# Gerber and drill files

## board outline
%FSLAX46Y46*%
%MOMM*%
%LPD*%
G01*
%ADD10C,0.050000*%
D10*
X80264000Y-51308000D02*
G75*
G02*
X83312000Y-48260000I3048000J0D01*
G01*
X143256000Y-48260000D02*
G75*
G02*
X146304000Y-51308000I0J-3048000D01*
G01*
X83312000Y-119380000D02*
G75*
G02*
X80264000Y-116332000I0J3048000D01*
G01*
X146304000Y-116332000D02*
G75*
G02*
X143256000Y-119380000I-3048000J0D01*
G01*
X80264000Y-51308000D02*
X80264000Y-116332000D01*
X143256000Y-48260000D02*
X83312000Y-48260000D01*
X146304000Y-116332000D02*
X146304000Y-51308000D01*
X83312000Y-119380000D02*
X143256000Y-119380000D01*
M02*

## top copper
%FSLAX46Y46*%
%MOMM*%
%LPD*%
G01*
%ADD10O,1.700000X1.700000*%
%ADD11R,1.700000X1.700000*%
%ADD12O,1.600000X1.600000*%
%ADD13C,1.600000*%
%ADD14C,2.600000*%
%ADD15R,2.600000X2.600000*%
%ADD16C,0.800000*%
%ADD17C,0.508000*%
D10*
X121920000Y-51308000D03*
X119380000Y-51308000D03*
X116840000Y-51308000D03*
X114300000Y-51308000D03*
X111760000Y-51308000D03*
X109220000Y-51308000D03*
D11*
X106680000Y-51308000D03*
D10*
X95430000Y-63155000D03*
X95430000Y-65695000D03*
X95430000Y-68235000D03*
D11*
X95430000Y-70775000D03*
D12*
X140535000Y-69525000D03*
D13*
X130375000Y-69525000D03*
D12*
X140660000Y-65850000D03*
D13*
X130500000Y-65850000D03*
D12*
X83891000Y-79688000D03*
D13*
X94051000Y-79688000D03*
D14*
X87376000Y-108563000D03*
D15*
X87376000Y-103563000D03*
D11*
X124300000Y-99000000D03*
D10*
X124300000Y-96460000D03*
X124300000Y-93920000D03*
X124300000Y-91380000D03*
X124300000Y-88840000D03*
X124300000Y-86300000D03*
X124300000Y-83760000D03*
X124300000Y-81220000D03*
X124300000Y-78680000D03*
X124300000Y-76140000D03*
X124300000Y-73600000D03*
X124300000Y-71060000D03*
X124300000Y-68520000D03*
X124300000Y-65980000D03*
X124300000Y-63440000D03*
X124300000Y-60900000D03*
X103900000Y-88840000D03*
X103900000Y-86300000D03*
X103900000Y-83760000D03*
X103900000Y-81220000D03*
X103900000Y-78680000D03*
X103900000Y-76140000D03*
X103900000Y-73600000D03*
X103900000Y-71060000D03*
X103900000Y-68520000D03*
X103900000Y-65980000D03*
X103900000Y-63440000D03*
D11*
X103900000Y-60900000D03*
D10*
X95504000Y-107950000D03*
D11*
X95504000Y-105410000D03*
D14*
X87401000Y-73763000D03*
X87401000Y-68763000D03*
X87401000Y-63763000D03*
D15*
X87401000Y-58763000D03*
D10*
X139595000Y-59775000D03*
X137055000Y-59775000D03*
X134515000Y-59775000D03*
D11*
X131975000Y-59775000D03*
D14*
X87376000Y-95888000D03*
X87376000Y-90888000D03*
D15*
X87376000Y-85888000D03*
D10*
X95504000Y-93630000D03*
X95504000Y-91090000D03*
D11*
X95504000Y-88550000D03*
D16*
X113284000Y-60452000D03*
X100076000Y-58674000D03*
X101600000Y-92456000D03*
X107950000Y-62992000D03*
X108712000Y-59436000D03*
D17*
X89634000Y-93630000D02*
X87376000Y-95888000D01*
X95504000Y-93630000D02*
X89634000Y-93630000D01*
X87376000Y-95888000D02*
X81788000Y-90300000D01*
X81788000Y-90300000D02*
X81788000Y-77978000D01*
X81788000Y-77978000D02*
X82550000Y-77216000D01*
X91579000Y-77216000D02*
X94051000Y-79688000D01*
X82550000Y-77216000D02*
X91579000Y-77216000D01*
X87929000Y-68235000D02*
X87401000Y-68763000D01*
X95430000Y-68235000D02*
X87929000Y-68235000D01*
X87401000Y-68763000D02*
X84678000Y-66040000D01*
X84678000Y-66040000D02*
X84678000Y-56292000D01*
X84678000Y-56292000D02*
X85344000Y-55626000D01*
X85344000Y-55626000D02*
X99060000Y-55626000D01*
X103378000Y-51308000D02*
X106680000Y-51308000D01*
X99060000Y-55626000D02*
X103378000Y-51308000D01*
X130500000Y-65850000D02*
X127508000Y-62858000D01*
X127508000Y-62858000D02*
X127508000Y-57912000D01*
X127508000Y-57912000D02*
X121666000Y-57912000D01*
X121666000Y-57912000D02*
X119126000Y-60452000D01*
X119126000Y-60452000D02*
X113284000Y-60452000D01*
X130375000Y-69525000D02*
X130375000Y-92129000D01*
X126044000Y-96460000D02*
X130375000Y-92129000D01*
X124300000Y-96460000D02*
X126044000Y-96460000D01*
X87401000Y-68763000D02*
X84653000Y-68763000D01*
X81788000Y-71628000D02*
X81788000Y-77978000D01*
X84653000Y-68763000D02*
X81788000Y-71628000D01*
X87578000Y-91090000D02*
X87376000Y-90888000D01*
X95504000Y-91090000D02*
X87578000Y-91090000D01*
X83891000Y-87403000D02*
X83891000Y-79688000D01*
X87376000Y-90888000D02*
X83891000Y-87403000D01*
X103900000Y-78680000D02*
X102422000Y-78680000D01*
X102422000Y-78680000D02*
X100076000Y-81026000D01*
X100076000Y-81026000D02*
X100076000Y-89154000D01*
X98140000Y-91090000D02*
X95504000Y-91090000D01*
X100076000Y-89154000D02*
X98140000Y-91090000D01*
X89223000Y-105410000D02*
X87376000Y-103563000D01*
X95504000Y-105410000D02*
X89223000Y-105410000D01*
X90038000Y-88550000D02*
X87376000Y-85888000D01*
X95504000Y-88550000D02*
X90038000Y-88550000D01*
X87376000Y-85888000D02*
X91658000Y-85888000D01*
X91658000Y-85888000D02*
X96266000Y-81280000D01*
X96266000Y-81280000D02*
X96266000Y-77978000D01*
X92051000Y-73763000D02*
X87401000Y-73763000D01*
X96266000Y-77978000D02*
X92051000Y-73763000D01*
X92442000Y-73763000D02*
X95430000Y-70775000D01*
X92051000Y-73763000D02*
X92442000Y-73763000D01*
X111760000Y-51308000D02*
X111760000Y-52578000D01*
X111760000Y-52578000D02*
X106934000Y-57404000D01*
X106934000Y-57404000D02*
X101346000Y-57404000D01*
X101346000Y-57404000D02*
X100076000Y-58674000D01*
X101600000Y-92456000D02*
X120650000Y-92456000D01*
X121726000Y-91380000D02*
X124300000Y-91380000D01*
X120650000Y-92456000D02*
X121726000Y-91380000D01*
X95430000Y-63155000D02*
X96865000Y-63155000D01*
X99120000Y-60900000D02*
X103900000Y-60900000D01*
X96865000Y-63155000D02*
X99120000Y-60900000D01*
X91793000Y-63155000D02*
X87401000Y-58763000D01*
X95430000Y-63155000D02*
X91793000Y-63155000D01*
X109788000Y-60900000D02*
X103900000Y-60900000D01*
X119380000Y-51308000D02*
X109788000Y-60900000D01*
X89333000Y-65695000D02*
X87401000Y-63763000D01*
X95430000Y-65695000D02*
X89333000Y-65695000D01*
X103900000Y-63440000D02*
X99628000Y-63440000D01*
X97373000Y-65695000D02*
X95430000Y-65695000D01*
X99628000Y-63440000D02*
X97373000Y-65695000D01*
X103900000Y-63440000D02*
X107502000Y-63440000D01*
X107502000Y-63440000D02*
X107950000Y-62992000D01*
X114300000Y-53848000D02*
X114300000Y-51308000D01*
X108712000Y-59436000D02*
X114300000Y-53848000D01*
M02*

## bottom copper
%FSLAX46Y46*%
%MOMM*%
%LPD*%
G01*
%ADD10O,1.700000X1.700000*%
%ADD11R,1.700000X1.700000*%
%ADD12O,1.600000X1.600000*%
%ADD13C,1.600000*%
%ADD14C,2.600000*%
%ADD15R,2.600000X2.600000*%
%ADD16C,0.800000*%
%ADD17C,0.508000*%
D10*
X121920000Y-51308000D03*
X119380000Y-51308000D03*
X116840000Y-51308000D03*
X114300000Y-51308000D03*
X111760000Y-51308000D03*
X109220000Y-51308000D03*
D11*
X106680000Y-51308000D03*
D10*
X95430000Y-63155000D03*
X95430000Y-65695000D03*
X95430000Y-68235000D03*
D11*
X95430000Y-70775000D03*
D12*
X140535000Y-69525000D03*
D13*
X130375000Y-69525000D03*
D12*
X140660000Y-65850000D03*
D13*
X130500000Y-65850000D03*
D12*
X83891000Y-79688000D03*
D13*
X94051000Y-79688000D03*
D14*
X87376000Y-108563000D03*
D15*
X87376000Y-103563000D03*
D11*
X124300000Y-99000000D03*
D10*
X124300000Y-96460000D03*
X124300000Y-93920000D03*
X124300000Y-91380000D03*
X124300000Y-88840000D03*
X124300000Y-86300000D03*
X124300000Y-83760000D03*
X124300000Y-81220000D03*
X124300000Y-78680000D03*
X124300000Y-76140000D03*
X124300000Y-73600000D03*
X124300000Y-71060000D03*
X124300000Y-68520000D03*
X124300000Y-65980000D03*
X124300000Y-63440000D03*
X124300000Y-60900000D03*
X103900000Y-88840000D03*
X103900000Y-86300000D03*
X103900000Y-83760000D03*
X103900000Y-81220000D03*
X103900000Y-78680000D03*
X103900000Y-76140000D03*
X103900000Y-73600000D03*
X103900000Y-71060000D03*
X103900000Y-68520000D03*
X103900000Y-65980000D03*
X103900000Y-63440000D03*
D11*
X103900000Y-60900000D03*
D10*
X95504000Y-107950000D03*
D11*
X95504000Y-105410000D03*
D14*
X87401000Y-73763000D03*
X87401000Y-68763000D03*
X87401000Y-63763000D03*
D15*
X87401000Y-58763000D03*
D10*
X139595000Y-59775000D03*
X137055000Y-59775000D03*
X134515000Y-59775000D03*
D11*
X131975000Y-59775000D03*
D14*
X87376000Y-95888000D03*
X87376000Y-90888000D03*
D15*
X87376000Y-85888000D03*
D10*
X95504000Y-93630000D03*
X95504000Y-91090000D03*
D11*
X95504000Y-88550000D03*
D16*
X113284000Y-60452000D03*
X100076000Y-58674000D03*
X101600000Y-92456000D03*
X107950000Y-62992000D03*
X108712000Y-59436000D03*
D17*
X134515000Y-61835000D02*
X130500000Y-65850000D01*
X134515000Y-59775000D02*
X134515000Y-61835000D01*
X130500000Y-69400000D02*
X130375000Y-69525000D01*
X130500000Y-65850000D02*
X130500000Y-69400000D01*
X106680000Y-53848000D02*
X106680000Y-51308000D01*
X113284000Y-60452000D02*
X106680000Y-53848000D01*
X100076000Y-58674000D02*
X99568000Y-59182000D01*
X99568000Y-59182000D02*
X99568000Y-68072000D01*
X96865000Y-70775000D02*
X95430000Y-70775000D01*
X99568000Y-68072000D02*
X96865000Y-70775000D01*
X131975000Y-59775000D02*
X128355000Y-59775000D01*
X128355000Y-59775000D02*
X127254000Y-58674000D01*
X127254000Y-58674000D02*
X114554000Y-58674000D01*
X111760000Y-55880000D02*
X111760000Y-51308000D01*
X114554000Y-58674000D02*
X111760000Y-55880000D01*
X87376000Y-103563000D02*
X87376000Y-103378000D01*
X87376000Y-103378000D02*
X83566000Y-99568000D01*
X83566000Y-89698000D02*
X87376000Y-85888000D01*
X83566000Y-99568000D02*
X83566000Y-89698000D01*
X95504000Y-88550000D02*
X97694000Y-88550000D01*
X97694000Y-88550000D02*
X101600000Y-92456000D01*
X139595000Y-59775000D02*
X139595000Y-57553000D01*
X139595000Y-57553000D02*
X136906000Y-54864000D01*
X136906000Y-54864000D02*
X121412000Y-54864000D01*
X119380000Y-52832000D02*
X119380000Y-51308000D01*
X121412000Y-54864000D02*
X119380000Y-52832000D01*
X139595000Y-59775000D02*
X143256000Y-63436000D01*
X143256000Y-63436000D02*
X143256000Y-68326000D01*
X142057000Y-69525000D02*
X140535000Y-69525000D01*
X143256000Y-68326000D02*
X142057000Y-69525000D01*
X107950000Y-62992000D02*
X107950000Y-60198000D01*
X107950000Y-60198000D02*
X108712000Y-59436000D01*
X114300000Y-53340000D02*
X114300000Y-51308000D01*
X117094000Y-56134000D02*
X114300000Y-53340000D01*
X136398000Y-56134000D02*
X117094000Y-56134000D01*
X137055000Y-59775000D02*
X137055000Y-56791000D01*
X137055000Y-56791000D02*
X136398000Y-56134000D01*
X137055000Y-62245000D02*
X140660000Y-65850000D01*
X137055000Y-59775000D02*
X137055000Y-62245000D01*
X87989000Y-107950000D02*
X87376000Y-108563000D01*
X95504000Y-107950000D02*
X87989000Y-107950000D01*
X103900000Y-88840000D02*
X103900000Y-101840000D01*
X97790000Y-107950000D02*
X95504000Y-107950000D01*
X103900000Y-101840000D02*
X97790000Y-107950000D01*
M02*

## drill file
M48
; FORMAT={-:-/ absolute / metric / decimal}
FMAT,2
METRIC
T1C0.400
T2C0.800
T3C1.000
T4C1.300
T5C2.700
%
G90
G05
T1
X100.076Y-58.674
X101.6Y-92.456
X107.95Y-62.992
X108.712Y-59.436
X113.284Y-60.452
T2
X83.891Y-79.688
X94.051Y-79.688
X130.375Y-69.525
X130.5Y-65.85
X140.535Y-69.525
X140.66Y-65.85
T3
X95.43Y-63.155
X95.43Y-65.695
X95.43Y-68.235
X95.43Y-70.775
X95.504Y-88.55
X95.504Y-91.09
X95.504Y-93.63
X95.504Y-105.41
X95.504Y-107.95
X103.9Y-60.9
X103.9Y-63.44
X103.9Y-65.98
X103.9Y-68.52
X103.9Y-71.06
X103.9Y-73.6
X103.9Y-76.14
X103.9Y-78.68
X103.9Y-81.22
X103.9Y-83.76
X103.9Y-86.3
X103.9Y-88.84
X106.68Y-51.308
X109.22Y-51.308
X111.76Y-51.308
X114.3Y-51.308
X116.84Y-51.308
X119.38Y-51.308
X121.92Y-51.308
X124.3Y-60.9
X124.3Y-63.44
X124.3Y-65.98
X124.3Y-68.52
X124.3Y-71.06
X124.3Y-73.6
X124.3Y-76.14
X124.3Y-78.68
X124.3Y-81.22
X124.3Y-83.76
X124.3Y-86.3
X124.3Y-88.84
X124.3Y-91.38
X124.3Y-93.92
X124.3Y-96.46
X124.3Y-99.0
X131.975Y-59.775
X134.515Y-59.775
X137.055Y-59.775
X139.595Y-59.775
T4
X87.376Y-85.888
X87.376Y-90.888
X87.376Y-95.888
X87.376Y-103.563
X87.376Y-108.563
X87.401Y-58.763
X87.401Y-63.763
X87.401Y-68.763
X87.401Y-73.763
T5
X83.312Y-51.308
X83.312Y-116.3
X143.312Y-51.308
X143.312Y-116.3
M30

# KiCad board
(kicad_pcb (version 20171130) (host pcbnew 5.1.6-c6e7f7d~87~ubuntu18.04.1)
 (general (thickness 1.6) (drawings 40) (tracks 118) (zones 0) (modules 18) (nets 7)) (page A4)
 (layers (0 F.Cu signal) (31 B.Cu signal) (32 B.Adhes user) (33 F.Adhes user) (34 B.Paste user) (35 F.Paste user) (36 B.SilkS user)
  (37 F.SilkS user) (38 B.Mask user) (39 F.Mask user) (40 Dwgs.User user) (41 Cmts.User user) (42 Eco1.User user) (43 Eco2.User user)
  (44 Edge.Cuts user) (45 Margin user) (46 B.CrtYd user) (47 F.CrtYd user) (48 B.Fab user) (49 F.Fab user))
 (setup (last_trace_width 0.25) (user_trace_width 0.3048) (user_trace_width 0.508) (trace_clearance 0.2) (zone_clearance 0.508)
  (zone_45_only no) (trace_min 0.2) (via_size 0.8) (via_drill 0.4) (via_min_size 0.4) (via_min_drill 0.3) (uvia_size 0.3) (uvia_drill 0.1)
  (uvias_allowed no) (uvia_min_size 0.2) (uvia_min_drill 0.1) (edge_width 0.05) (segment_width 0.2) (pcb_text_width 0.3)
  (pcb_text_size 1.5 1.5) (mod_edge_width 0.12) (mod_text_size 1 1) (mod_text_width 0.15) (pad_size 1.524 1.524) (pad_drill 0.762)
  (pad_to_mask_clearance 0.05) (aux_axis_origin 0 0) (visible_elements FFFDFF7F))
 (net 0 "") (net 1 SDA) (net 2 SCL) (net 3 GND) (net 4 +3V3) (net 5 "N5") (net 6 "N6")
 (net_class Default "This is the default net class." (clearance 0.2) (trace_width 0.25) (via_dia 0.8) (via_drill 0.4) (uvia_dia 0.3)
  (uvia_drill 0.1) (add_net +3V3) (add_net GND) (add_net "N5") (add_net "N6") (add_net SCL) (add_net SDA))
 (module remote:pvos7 (layer F.Cu) (at 135.89 91.948 90)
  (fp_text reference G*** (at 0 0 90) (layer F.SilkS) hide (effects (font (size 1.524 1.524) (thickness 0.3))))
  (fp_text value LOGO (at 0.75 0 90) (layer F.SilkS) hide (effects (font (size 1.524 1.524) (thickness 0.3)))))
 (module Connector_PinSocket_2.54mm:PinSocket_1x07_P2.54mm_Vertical (layer F.Cu) (at 106.68 51.308 90)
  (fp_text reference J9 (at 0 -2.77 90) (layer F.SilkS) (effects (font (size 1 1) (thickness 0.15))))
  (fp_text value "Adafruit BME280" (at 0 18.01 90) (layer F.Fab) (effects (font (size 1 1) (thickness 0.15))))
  (pad 7 thru_hole oval (at 0 15.24 90) (size 1.7 1.7) (drill 1) (layers *.Cu *.Mask))
  (pad 6 thru_hole oval (at 0 12.7 90) (size 1.7 1.7) (drill 1) (layers *.Cu *.Mask) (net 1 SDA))
  (pad 5 thru_hole oval (at 0 10.16 90) (size 1.7 1.7) (drill 1) (layers *.Cu *.Mask))
  (pad 4 thru_hole oval (at 0 7.62 90) (size 1.7 1.7) (drill 1) (layers *.Cu *.Mask) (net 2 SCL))
  (pad 3 thru_hole oval (at 0 5.08 90) (size 1.7 1.7) (drill 1) (layers *.Cu *.Mask) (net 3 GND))
  (pad 2 thru_hole oval (at 0 2.54 90) (size 1.7 1.7) (drill 1) (layers *.Cu *.Mask))
  (pad 1 thru_hole rect (at 0 0 90) (size 1.7 1.7) (drill 1) (layers *.Cu *.Mask) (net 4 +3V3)))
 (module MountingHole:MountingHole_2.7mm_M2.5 (layer F.Cu) (at 143.312 116.3)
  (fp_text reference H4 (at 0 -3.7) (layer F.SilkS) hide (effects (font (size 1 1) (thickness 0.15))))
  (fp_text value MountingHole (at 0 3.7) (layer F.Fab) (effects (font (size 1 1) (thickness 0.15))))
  (pad 1 np_thru_hole circle (at 0 0) (size 2.7 2.7) (drill 2.7) (layers *.Cu *.Mask)))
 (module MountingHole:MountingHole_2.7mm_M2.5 (layer F.Cu) (at 83.312 116.3)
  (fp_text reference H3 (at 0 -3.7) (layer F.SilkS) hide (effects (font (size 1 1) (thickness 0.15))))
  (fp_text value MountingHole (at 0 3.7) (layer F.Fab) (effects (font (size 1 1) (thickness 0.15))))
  (pad 1 np_thru_hole circle (at 0 0) (size 2.7 2.7) (drill 2.7) (layers *.Cu *.Mask)))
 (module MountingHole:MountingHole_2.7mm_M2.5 (layer F.Cu) (at 143.312 51.308)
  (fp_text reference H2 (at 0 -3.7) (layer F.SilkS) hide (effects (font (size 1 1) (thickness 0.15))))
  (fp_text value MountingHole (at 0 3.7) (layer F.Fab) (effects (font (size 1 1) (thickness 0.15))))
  (pad 1 np_thru_hole circle (at 0 0) (size 2.7 2.7) (drill 2.7) (layers *.Cu *.Mask)))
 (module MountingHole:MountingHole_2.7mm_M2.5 (layer F.Cu) (at 83.312 51.308)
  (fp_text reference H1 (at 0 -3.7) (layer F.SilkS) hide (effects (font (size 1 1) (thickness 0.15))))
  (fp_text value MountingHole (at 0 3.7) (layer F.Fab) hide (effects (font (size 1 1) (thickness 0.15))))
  (pad 1 np_thru_hole circle (at 0 0) (size 2.7 2.7) (drill 2.7) (layers *.Cu *.Mask)))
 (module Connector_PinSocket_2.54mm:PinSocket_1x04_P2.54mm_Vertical (layer F.Cu) (at 95.43 70.775 180)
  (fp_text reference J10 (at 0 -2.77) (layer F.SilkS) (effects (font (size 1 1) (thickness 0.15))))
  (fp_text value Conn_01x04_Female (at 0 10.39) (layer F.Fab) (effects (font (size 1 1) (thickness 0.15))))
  (pad 4 thru_hole oval (at 0 7.62 180) (size 1.7 1.7) (drill 1) (layers *.Cu *.Mask) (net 1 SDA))
  (pad 3 thru_hole oval (at 0 5.08 180) (size 1.7 1.7) (drill 1) (layers *.Cu *.Mask) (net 2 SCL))
  (pad 2 thru_hole oval (at 0 2.54 180) (size 1.7 1.7) (drill 1) (layers *.Cu *.Mask) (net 4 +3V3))
  (pad 1 thru_hole rect (at 0 0 180) (size 1.7 1.7) (drill 1) (layers *.Cu *.Mask) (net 3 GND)))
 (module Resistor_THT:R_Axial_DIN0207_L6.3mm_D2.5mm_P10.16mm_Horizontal (layer F.Cu) (at 130.375 69.525)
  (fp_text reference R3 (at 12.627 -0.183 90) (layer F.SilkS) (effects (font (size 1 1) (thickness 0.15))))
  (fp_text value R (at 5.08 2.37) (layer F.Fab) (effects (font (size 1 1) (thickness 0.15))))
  (pad 2 thru_hole oval (at 10.16 0) (size 1.6 1.6) (drill 0.8) (layers *.Cu *.Mask) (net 1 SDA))
  (pad 1 thru_hole circle (at 0 0) (size 1.6 1.6) (drill 0.8) (layers *.Cu *.Mask) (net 4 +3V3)))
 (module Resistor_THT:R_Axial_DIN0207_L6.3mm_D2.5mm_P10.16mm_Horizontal (layer F.Cu) (at 130.5 65.85)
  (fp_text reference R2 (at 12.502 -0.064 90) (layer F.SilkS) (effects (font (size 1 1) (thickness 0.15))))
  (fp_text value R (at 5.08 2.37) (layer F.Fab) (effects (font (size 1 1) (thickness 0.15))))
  (pad 2 thru_hole oval (at 10.16 0) (size 1.6 1.6) (drill 0.8) (layers *.Cu *.Mask) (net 2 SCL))
  (pad 1 thru_hole circle (at 0 0) (size 1.6 1.6) (drill 0.8) (layers *.Cu *.Mask) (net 4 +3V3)))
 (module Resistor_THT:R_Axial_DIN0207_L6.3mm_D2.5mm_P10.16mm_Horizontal (layer F.Cu) (at 94.051 79.688 180)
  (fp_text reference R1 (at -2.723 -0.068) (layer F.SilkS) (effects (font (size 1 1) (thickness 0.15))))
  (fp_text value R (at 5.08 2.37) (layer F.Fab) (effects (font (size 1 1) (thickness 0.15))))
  (pad 2 thru_hole oval (at 10.16 0 180) (size 1.6 1.6) (drill 0.8) (layers *.Cu *.Mask) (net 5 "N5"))
  (pad 1 thru_hole circle (at 0 0 180) (size 1.6 1.6) (drill 0.8) (layers *.Cu *.Mask) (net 4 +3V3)))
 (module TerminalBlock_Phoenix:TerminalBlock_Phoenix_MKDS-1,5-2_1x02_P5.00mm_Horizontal (layer F.Cu) (at 87.376 103.563 270)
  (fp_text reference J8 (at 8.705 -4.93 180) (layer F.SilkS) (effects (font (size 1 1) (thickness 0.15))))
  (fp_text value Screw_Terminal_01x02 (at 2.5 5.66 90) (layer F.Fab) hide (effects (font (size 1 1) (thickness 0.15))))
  (pad 2 thru_hole circle (at 5 0 270) (size 2.6 2.6) (drill 1.3) (layers *.Cu *.Mask) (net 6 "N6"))
  (pad 1 thru_hole rect (at 0 0 270) (size 2.6 2.6) (drill 1.3) (layers *.Cu *.Mask) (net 3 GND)))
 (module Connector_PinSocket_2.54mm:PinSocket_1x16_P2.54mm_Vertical (layer F.Cu) (at 124.3 99 180)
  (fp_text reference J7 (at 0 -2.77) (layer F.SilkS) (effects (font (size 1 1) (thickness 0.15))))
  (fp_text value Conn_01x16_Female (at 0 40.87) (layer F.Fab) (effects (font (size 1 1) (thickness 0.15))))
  (pad 1 thru_hole rect (at 0 0 180) (size 1.7 1.7) (drill 1) (layers *.Cu *.Mask))
  (pad 2 thru_hole oval (at 0 2.54 180) (size 1.7 1.7) (drill 1) (layers *.Cu *.Mask) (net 4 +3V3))
  (pad 3 thru_hole oval (at 0 5.08 180) (size 1.7 1.7) (drill 1) (layers *.Cu *.Mask))
  (pad 4 thru_hole oval (at 0 7.62 180) (size 1.7 1.7) (drill 1) (layers *.Cu *.Mask) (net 3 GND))
  (pad 5 thru_hole oval (at 0 10.16 180) (size 1.7 1.7) (drill 1) (layers *.Cu *.Mask))
  (pad 6 thru_hole oval (at 0 12.7 180) (size 1.7 1.7) (drill 1) (layers *.Cu *.Mask))
  (pad 7 thru_hole oval (at 0 15.24 180) (size 1.7 1.7) (drill 1) (layers *.Cu *.Mask))
  (pad 8 thru_hole oval (at 0 17.78 180) (size 1.7 1.7) (drill 1) (layers *.Cu *.Mask))
  (pad 9 thru_hole oval (at 0 20.32 180) (size 1.7 1.7) (drill 1) (layers *.Cu *.Mask))
  (pad 10 thru_hole oval (at 0 22.86 180) (size 1.7 1.7) (drill 1) (layers *.Cu *.Mask))
  (pad 11 thru_hole oval (at 0 25.4 180) (size 1.7 1.7) (drill 1) (layers *.Cu *.Mask))
  (pad 12 thru_hole oval (at 0 27.94 180) (size 1.7 1.7) (drill 1) (layers *.Cu *.Mask))
  (pad 13 thru_hole oval (at 0 30.48 180) (size 1.7 1.7) (drill 1) (layers *.Cu *.Mask))
  (pad 14 thru_hole oval (at 0 33.02 180) (size 1.7 1.7) (drill 1) (layers *.Cu *.Mask))
  (pad 15 thru_hole oval (at 0 35.56 180) (size 1.7 1.7) (drill 1) (layers *.Cu *.Mask))
  (pad 16 thru_hole oval (at 0 38.1 180) (size 1.7 1.7) (drill 1) (layers *.Cu *.Mask)))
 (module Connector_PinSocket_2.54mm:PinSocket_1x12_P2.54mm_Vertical (layer F.Cu) (at 103.9 60.9)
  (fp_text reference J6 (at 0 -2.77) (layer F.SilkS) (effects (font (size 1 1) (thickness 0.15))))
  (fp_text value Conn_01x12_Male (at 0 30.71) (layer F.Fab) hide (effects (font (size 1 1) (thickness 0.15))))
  (pad 12 thru_hole oval (at 0 27.94) (size 1.7 1.7) (drill 1) (layers *.Cu *.Mask) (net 6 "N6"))
  (pad 11 thru_hole oval (at 0 25.4) (size 1.7 1.7) (drill 1) (layers *.Cu *.Mask))
  (pad 10 thru_hole oval (at 0 22.86) (size 1.7 1.7) (drill 1) (layers *.Cu *.Mask))
  (pad 9 thru_hole oval (at 0 20.32) (size 1.7 1.7) (drill 1) (layers *.Cu *.Mask))
  (pad 8 thru_hole oval (at 0 17.78) (size 1.7 1.7) (drill 1) (layers *.Cu *.Mask) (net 5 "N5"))
  (pad 7 thru_hole oval (at 0 15.24) (size 1.7 1.7) (drill 1) (layers *.Cu *.Mask))
  (pad 6 thru_hole oval (at 0 12.7) (size 1.7 1.7) (drill 1) (layers *.Cu *.Mask))
  (pad 5 thru_hole oval (at 0 10.16) (size 1.7 1.7) (drill 1) (layers *.Cu *.Mask))
  (pad 4 thru_hole oval (at 0 7.62) (size 1.7 1.7) (drill 1) (layers *.Cu *.Mask))
  (pad 3 thru_hole oval (at 0 5.08) (size 1.7 1.7) (drill 1) (layers *.Cu *.Mask))
  (pad 2 thru_hole oval (at 0 2.54) (size 1.7 1.7) (drill 1) (layers *.Cu *.Mask) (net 2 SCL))
  (pad 1 thru_hole rect (at 0 0) (size 1.7 1.7) (drill 1) (layers *.Cu *.Mask) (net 1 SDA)))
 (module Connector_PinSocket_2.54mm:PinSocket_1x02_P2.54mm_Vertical (layer F.Cu) (at 95.504 105.41)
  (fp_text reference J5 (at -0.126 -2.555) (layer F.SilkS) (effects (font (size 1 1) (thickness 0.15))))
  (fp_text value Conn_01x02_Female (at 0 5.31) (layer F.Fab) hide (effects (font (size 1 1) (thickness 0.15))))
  (pad 2 thru_hole oval (at 0 2.54) (size 1.7 1.7) (drill 1) (layers *.Cu *.Mask) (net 6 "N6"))
  (pad 1 thru_hole rect (at 0 0) (size 1.7 1.7) (drill 1) (layers *.Cu *.Mask) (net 3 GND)))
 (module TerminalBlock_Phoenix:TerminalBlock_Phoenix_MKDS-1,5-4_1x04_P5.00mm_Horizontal (layer F.Cu) (at 87.401 58.763 270)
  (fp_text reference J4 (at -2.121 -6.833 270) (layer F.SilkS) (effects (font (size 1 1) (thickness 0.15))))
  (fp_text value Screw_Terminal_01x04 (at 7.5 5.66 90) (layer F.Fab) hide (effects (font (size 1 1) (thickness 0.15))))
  (pad 4 thru_hole circle (at 15 0 270) (size 2.6 2.6) (drill 1.3) (layers *.Cu *.Mask) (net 3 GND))
  (pad 3 thru_hole circle (at 10 0 270) (size 2.6 2.6) (drill 1.3) (layers *.Cu *.Mask) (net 4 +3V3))
  (pad 2 thru_hole circle (at 5 0 270) (size 2.6 2.6) (drill 1.3) (layers *.Cu *.Mask) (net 2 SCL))
  (pad 1 thru_hole rect (at 0 0 270) (size 2.6 2.6) (drill 1.3) (layers *.Cu *.Mask) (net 1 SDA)))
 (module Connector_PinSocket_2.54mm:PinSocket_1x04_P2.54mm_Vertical (layer F.Cu) (at 131.975 59.775 90)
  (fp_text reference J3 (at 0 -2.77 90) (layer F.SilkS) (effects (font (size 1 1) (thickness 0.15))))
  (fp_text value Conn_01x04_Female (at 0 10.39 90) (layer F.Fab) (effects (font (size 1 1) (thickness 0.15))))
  (pad 4 thru_hole oval (at 0 7.62 90) (size 1.7 1.7) (drill 1) (layers *.Cu *.Mask) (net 1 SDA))
  (pad 3 thru_hole oval (at 0 5.08 90) (size 1.7 1.7) (drill 1) (layers *.Cu *.Mask) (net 2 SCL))
  (pad 2 thru_hole oval (at 0 2.54 90) (size 1.7 1.7) (drill 1) (layers *.Cu *.Mask) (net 4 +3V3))
  (pad 1 thru_hole rect (at 0 0 90) (size 1.7 1.7) (drill 1) (layers *.Cu *.Mask) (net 3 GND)))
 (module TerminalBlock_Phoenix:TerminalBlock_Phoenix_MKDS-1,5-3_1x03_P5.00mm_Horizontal (layer F.Cu) (at 87.376 85.888 270)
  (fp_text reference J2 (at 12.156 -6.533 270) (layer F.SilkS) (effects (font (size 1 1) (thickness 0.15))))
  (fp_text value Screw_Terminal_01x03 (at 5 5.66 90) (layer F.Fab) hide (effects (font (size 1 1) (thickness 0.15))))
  (pad 3 thru_hole circle (at 10 0 270) (size 2.6 2.6) (drill 1.3) (layers *.Cu *.Mask) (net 4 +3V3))
  (pad 2 thru_hole circle (at 5 0 270) (size 2.6 2.6) (drill 1.3) (layers *.Cu *.Mask) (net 5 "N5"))
  (pad 1 thru_hole rect (at 0 0 270) (size 2.6 2.6) (drill 1.3) (layers *.Cu *.Mask) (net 3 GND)))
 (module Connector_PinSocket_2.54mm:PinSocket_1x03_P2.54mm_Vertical (layer F.Cu) (at 95.504 88.55)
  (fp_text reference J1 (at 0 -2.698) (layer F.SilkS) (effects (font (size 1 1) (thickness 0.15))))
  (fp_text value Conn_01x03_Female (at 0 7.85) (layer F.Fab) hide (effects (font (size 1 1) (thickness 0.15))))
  (pad 3 thru_hole oval (at 0 5.08) (size 1.7 1.7) (drill 1) (layers *.Cu *.Mask) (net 4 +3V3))
  (pad 2 thru_hole oval (at 0 2.54) (size 1.7 1.7) (drill 1) (layers *.Cu *.Mask) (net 5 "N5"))
  (pad 1 thru_hole rect (at 0 0) (size 1.7 1.7) (drill 1) (layers *.Cu *.Mask) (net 3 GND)))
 (gr_arc (start 83.312 51.308) (end 83.312 48.26) (angle -90) (layer Edge.Cuts) (width 0.05))
 (gr_arc (start 143.256 51.308) (end 146.304 51.308) (angle -90) (layer Edge.Cuts) (width 0.05))
 (gr_arc (start 83.312 116.332) (end 80.264 116.332) (angle -90) (layer Edge.Cuts) (width 0.05))
 (gr_arc (start 143.256 116.332) (end 143.256 119.38) (angle -90) (layer Edge.Cuts) (width 0.05))
 (gr_line (start 80.264 51.308) (end 80.264 116.332) (layer Edge.Cuts) (width 0.05))
 (gr_line (start 143.256 48.26) (end 83.312 48.26) (layer Edge.Cuts) (width 0.05))
 (gr_line (start 146.304 116.332) (end 146.304 51.308) (layer Edge.Cuts) (width 0.05))
 (gr_line (start 83.312 119.38) (end 143.256 119.38) (layer Edge.Cuts) (width 0.05))
 (segment (start 89.634 93.63) (end 87.376 95.888) (width 0.508) (layer F.Cu) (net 4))
 (segment (start 95.504 93.63) (end 89.634 93.63) (width 0.508) (layer F.Cu) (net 4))
 (segment (start 87.376 95.888) (end 81.788 90.3) (width 0.508) (layer F.Cu) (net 4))
 (segment (start 81.788 90.3) (end 81.788 77.978) (width 0.508) (layer F.Cu) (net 4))
 (segment (start 81.788 77.978) (end 82.55 77.216) (width 0.508) (layer F.Cu) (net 4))
 (segment (start 91.579 77.216) (end 94.051 79.688) (width 0.508) (layer F.Cu) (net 4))
 (segment (start 82.55 77.216) (end 91.579 77.216) (width 0.508) (layer F.Cu) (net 4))
 (segment (start 87.929 68.235) (end 87.401 68.763) (width 0.508) (layer F.Cu) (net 4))
 (segment (start 95.43 68.235) (end 87.929 68.235) (width 0.508) (layer F.Cu) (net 4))
 (segment (start 87.401 68.763) (end 84.678 66.04) (width 0.508) (layer F.Cu) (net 4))
 (segment (start 84.678 66.04) (end 84.678 56.292) (width 0.508) (layer F.Cu) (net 4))
 (segment (start 84.678 56.292) (end 85.344 55.626) (width 0.508) (layer F.Cu) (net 4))
 (segment (start 85.344 55.626) (end 99.06 55.626) (width 0.508) (layer F.Cu) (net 4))
 (segment (start 103.378 51.308) (end 106.68 51.308) (width 0.508) (layer F.Cu) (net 4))
 (segment (start 99.06 55.626) (end 103.378 51.308) (width 0.508) (layer F.Cu) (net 4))
 (segment (start 134.515 61.835) (end 130.5 65.85) (width 0.508) (layer B.Cu) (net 4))
 (segment (start 134.515 59.775) (end 134.515 61.835) (width 0.508) (layer B.Cu) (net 4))
 (segment (start 130.5 69.4) (end 130.375 69.525) (width 0.508) (layer B.Cu) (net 4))
 (segment (start 130.5 65.85) (end 130.5 69.4) (width 0.508) (layer B.Cu) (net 4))
 (segment (start 130.5 65.85) (end 127.508 62.858) (width 0.508) (layer F.Cu) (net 4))
 (segment (start 127.508 62.858) (end 127.508 57.912) (width 0.508) (layer F.Cu) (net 4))
 (segment (start 127.508 57.912) (end 121.666 57.912) (width 0.508) (layer F.Cu) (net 4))
 (via (at 113.284 60.452) (size 0.8) (drill 0.4) (layers F.Cu B.Cu) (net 4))
 (segment (start 121.666 57.912) (end 119.126 60.452) (width 0.508) (layer F.Cu) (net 4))
 (segment (start 119.126 60.452) (end 113.284 60.452) (width 0.508) (layer F.Cu) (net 4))
 (segment (start 106.68 53.848) (end 106.68 51.308) (width 0.508) (layer B.Cu) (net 4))
 (segment (start 113.284 60.452) (end 106.68 53.848) (width 0.508) (layer B.Cu) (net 4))
 (segment (start 130.375 69.525) (end 130.375 92.129) (width 0.508) (layer F.Cu) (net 4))
 (segment (start 126.044 96.46) (end 130.375 92.129) (width 0.508) (layer F.Cu) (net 4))
 (segment (start 124.3 96.46) (end 126.044 96.46) (width 0.508) (layer F.Cu) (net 4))
 (segment (start 87.401 68.763) (end 84.653 68.763) (width 0.508) (layer F.Cu) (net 4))
 (segment (start 81.788 71.628) (end 81.788 77.978) (width 0.508) (layer F.Cu) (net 4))
 (segment (start 84.653 68.763) (end 81.788 71.628) (width 0.508) (layer F.Cu) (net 4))
 (segment (start 87.578 91.09) (end 87.376 90.888) (width 0.508) (layer F.Cu) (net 5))
 (segment (start 95.504 91.09) (end 87.578 91.09) (width 0.508) (layer F.Cu) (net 5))
 (segment (start 83.891 87.403) (end 83.891 79.688) (width 0.508) (layer F.Cu) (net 5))
 (segment (start 87.376 90.888) (end 83.891 87.403) (width 0.508) (layer F.Cu) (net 5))
 (segment (start 103.9 78.68) (end 102.422 78.68) (width 0.508) (layer F.Cu) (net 5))
 (segment (start 102.422 78.68) (end 100.076 81.026) (width 0.508) (layer F.Cu) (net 5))
 (segment (start 100.076 81.026) (end 100.076 89.154) (width 0.508) (layer F.Cu) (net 5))
 (segment (start 98.14 91.09) (end 95.504 91.09) (width 0.508) (layer F.Cu) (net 5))
 (segment (start 100.076 89.154) (end 98.14 91.09) (width 0.508) (layer F.Cu) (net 5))
 (segment (start 89.223 105.41) (end 87.376 103.563) (width 0.508) (layer F.Cu) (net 3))
 (segment (start 95.504 105.41) (end 89.223 105.41) (width 0.508) (layer F.Cu) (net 3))
 (segment (start 90.038 88.55) (end 87.376 85.888) (width 0.508) (layer F.Cu) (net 3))
 (segment (start 95.504 88.55) (end 90.038 88.55) (width 0.508) (layer F.Cu) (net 3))
 (segment (start 87.376 85.888) (end 91.658 85.888) (width 0.508) (layer F.Cu) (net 3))
 (segment (start 91.658 85.888) (end 96.266 81.28) (width 0.508) (layer F.Cu) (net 3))
 (segment (start 96.266 81.28) (end 96.266 77.978) (width 0.508) (layer F.Cu) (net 3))
 (segment (start 92.051 73.763) (end 87.401 73.763) (width 0.508) (layer F.Cu) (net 3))
 (segment (start 96.266 77.978) (end 92.051 73.763) (width 0.508) (layer F.Cu) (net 3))
 (segment (start 92.442 73.763) (end 95.43 70.775) (width 0.508) (layer F.Cu) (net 3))
 (segment (start 92.051 73.763) (end 92.442 73.763) (width 0.508) (layer F.Cu) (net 3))
 (segment (start 111.76 51.308) (end 111.76 52.578) (width 0.508) (layer F.Cu) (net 3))
 (segment (start 111.76 52.578) (end 106.934 57.404) (width 0.508) (layer F.Cu) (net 3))
 (via (at 100.076 58.674) (size 0.8) (drill 0.4) (layers F.Cu B.Cu) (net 3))
 (segment (start 106.934 57.404) (end 101.346 57.404) (width 0.508) (layer F.Cu) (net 3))
 (segment (start 101.346 57.404) (end 100.076 58.674) (width 0.508) (layer F.Cu) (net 3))
 (segment (start 100.076 58.674) (end 99.568 59.182) (width 0.508) (layer B.Cu) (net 3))
 (segment (start 99.568 59.182) (end 99.568 68.072) (width 0.508) (layer B.Cu) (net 3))
 (segment (start 96.865 70.775) (end 95.43 70.775) (width 0.508) (layer B.Cu) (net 3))
 (segment (start 99.568 68.072) (end 96.865 70.775) (width 0.508) (layer B.Cu) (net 3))
 (segment (start 131.975 59.775) (end 128.355 59.775) (width 0.508) (layer B.Cu) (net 3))
 (segment (start 128.355 59.775) (end 127.254 58.674) (width 0.508) (layer B.Cu) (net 3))
 (segment (start 127.254 58.674) (end 114.554 58.674) (width 0.508) (layer B.Cu) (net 3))
 (segment (start 111.76 55.88) (end 111.76 51.308) (width 0.508) (layer B.Cu) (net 3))
 (segment (start 114.554 58.674) (end 111.76 55.88) (width 0.508) (layer B.Cu) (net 3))
 (segment (start 87.376 103.563) (end 87.376 103.378) (width 0.508) (layer B.Cu) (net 3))
 (segment (start 87.376 103.378) (end 83.566 99.568) (width 0.508) (layer B.Cu) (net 3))
 (segment (start 83.566 89.698) (end 87.376 85.888) (width 0.508) (layer B.Cu) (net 3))
 (segment (start 83.566 99.568) (end 83.566 89.698) (width 0.508) (layer B.Cu) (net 3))
 (segment (start 95.504 88.55) (end 97.694 88.55) (width 0.508) (layer B.Cu) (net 3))
 (segment (start 97.694 88.55) (end 101.6 92.456) (width 0.508) (layer B.Cu) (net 3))
 (via (at 101.6 92.456) (size 0.8) (drill 0.4) (layers F.Cu B.Cu) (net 3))
 (segment (start 101.6 92.456) (end 120.65 92.456) (width 0.508) (layer F.Cu) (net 3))
 (segment (start 121.726 91.38) (end 124.3 91.38) (width 0.508) (layer F.Cu) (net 3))
 (segment (start 120.65 92.456) (end 121.726 91.38) (width 0.508) (layer F.Cu) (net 3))
 (segment (start 95.43 63.155) (end 96.865 63.155) (width 0.508) (layer F.Cu) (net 1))
 (segment (start 99.12 60.9) (end 103.9 60.9) (width 0.508) (layer F.Cu) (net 1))
 (segment (start 96.865 63.155) (end 99.12 60.9) (width 0.508) (layer F.Cu) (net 1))
 (segment (start 91.793 63.155) (end 87.401 58.763) (width 0.508) (layer F.Cu) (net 1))
 (segment (start 95.43 63.155) (end 91.793 63.155) (width 0.508) (layer F.Cu) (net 1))
 (segment (start 109.788 60.9) (end 103.9 60.9) (width 0.508) (layer F.Cu) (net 1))
 (segment (start 119.38 51.308) (end 109.788 60.9) (width 0.508) (layer F.Cu) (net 1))
 (segment (start 139.595 59.775) (end 139.595 57.553) (width 0.508) (layer B.Cu) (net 1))
 (segment (start 139.595 57.553) (end 136.906 54.864) (width 0.508) (layer B.Cu) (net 1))
 (segment (start 136.906 54.864) (end 121.412 54.864) (width 0.508) (layer B.Cu) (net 1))
 (segment (start 119.38 52.832) (end 119.38 51.308) (width 0.508) (layer B.Cu) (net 1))
 (segment (start 121.412 54.864) (end 119.38 52.832) (width 0.508) (layer B.Cu) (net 1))
 (segment (start 139.595 59.775) (end 143.256 63.436) (width 0.508) (layer B.Cu) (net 1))
 (segment (start 143.256 63.436) (end 143.256 68.326) (width 0.508) (layer B.Cu) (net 1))
 (segment (start 142.057 69.525) (end 140.535 69.525) (width 0.508) (layer B.Cu) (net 1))
 (segment (start 143.256 68.326) (end 142.057 69.525) (width 0.508) (layer B.Cu) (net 1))
 (segment (start 89.333 65.695) (end 87.401 63.763) (width 0.508) (layer F.Cu) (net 2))
 (segment (start 95.43 65.695) (end 89.333 65.695) (width 0.508) (layer F.Cu) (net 2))
 (segment (start 103.9 63.44) (end 99.628 63.44) (width 0.508) (layer F.Cu) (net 2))
 (segment (start 97.373 65.695) (end 95.43 65.695) (width 0.508) (layer F.Cu) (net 2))
 (segment (start 99.628 63.44) (end 97.373 65.695) (width 0.508) (layer F.Cu) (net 2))
 (via (at 107.95 62.992) (size 0.8) (drill 0.4) (layers F.Cu B.Cu) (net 2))
 (segment (start 103.9 63.44) (end 107.502 63.44) (width 0.508) (layer F.Cu) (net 2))
 (segment (start 107.502 63.44) (end 107.95 62.992) (width 0.508) (layer F.Cu) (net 2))
 (via (at 108.712 59.436) (size 0.8) (drill 0.4) (layers F.Cu B.Cu) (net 2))
 (segment (start 107.95 62.992) (end 107.95 60.198) (width 0.508) (layer B.Cu) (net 2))
 (segment (start 107.95 60.198) (end 108.712 59.436) (width 0.508) (layer B.Cu) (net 2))
 (segment (start 114.3 53.848) (end 114.3 51.308) (width 0.508) (layer F.Cu) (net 2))
 (segment (start 108.712 59.436) (end 114.3 53.848) (width 0.508) (layer F.Cu) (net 2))
 (segment (start 114.3 53.34) (end 114.3 51.308) (width 0.508) (layer B.Cu) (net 2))
 (segment (start 117.094 56.134) (end 114.3 53.34) (width 0.508) (layer B.Cu) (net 2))
 (segment (start 136.398 56.134) (end 117.094 56.134) (width 0.508) (layer B.Cu) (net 2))
 (segment (start 137.055 59.775) (end 137.055 56.791) (width 0.508) (layer B.Cu) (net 2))
 (segment (start 137.055 56.791) (end 136.398 56.134) (width 0.508) (layer B.Cu) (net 2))
 (segment (start 137.055 62.245) (end 140.66 65.85) (width 0.508) (layer B.Cu) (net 2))
 (segment (start 137.055 59.775) (end 137.055 62.245) (width 0.508) (layer B.Cu) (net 2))
 (segment (start 87.989 107.95) (end 87.376 108.563) (width 0.508) (layer B.Cu) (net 6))
 (segment (start 95.504 107.95) (end 87.989 107.95) (width 0.508) (layer B.Cu) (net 6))
 (segment (start 103.9 88.84) (end 103.9 101.84) (width 0.508) (layer B.Cu) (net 6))
 (segment (start 97.79 107.95) (end 95.504 107.95) (width 0.508) (layer B.Cu) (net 6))
 (segment (start 103.9 101.84) (end 97.79 107.95) (width 0.508) (layer B.Cu) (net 6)))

